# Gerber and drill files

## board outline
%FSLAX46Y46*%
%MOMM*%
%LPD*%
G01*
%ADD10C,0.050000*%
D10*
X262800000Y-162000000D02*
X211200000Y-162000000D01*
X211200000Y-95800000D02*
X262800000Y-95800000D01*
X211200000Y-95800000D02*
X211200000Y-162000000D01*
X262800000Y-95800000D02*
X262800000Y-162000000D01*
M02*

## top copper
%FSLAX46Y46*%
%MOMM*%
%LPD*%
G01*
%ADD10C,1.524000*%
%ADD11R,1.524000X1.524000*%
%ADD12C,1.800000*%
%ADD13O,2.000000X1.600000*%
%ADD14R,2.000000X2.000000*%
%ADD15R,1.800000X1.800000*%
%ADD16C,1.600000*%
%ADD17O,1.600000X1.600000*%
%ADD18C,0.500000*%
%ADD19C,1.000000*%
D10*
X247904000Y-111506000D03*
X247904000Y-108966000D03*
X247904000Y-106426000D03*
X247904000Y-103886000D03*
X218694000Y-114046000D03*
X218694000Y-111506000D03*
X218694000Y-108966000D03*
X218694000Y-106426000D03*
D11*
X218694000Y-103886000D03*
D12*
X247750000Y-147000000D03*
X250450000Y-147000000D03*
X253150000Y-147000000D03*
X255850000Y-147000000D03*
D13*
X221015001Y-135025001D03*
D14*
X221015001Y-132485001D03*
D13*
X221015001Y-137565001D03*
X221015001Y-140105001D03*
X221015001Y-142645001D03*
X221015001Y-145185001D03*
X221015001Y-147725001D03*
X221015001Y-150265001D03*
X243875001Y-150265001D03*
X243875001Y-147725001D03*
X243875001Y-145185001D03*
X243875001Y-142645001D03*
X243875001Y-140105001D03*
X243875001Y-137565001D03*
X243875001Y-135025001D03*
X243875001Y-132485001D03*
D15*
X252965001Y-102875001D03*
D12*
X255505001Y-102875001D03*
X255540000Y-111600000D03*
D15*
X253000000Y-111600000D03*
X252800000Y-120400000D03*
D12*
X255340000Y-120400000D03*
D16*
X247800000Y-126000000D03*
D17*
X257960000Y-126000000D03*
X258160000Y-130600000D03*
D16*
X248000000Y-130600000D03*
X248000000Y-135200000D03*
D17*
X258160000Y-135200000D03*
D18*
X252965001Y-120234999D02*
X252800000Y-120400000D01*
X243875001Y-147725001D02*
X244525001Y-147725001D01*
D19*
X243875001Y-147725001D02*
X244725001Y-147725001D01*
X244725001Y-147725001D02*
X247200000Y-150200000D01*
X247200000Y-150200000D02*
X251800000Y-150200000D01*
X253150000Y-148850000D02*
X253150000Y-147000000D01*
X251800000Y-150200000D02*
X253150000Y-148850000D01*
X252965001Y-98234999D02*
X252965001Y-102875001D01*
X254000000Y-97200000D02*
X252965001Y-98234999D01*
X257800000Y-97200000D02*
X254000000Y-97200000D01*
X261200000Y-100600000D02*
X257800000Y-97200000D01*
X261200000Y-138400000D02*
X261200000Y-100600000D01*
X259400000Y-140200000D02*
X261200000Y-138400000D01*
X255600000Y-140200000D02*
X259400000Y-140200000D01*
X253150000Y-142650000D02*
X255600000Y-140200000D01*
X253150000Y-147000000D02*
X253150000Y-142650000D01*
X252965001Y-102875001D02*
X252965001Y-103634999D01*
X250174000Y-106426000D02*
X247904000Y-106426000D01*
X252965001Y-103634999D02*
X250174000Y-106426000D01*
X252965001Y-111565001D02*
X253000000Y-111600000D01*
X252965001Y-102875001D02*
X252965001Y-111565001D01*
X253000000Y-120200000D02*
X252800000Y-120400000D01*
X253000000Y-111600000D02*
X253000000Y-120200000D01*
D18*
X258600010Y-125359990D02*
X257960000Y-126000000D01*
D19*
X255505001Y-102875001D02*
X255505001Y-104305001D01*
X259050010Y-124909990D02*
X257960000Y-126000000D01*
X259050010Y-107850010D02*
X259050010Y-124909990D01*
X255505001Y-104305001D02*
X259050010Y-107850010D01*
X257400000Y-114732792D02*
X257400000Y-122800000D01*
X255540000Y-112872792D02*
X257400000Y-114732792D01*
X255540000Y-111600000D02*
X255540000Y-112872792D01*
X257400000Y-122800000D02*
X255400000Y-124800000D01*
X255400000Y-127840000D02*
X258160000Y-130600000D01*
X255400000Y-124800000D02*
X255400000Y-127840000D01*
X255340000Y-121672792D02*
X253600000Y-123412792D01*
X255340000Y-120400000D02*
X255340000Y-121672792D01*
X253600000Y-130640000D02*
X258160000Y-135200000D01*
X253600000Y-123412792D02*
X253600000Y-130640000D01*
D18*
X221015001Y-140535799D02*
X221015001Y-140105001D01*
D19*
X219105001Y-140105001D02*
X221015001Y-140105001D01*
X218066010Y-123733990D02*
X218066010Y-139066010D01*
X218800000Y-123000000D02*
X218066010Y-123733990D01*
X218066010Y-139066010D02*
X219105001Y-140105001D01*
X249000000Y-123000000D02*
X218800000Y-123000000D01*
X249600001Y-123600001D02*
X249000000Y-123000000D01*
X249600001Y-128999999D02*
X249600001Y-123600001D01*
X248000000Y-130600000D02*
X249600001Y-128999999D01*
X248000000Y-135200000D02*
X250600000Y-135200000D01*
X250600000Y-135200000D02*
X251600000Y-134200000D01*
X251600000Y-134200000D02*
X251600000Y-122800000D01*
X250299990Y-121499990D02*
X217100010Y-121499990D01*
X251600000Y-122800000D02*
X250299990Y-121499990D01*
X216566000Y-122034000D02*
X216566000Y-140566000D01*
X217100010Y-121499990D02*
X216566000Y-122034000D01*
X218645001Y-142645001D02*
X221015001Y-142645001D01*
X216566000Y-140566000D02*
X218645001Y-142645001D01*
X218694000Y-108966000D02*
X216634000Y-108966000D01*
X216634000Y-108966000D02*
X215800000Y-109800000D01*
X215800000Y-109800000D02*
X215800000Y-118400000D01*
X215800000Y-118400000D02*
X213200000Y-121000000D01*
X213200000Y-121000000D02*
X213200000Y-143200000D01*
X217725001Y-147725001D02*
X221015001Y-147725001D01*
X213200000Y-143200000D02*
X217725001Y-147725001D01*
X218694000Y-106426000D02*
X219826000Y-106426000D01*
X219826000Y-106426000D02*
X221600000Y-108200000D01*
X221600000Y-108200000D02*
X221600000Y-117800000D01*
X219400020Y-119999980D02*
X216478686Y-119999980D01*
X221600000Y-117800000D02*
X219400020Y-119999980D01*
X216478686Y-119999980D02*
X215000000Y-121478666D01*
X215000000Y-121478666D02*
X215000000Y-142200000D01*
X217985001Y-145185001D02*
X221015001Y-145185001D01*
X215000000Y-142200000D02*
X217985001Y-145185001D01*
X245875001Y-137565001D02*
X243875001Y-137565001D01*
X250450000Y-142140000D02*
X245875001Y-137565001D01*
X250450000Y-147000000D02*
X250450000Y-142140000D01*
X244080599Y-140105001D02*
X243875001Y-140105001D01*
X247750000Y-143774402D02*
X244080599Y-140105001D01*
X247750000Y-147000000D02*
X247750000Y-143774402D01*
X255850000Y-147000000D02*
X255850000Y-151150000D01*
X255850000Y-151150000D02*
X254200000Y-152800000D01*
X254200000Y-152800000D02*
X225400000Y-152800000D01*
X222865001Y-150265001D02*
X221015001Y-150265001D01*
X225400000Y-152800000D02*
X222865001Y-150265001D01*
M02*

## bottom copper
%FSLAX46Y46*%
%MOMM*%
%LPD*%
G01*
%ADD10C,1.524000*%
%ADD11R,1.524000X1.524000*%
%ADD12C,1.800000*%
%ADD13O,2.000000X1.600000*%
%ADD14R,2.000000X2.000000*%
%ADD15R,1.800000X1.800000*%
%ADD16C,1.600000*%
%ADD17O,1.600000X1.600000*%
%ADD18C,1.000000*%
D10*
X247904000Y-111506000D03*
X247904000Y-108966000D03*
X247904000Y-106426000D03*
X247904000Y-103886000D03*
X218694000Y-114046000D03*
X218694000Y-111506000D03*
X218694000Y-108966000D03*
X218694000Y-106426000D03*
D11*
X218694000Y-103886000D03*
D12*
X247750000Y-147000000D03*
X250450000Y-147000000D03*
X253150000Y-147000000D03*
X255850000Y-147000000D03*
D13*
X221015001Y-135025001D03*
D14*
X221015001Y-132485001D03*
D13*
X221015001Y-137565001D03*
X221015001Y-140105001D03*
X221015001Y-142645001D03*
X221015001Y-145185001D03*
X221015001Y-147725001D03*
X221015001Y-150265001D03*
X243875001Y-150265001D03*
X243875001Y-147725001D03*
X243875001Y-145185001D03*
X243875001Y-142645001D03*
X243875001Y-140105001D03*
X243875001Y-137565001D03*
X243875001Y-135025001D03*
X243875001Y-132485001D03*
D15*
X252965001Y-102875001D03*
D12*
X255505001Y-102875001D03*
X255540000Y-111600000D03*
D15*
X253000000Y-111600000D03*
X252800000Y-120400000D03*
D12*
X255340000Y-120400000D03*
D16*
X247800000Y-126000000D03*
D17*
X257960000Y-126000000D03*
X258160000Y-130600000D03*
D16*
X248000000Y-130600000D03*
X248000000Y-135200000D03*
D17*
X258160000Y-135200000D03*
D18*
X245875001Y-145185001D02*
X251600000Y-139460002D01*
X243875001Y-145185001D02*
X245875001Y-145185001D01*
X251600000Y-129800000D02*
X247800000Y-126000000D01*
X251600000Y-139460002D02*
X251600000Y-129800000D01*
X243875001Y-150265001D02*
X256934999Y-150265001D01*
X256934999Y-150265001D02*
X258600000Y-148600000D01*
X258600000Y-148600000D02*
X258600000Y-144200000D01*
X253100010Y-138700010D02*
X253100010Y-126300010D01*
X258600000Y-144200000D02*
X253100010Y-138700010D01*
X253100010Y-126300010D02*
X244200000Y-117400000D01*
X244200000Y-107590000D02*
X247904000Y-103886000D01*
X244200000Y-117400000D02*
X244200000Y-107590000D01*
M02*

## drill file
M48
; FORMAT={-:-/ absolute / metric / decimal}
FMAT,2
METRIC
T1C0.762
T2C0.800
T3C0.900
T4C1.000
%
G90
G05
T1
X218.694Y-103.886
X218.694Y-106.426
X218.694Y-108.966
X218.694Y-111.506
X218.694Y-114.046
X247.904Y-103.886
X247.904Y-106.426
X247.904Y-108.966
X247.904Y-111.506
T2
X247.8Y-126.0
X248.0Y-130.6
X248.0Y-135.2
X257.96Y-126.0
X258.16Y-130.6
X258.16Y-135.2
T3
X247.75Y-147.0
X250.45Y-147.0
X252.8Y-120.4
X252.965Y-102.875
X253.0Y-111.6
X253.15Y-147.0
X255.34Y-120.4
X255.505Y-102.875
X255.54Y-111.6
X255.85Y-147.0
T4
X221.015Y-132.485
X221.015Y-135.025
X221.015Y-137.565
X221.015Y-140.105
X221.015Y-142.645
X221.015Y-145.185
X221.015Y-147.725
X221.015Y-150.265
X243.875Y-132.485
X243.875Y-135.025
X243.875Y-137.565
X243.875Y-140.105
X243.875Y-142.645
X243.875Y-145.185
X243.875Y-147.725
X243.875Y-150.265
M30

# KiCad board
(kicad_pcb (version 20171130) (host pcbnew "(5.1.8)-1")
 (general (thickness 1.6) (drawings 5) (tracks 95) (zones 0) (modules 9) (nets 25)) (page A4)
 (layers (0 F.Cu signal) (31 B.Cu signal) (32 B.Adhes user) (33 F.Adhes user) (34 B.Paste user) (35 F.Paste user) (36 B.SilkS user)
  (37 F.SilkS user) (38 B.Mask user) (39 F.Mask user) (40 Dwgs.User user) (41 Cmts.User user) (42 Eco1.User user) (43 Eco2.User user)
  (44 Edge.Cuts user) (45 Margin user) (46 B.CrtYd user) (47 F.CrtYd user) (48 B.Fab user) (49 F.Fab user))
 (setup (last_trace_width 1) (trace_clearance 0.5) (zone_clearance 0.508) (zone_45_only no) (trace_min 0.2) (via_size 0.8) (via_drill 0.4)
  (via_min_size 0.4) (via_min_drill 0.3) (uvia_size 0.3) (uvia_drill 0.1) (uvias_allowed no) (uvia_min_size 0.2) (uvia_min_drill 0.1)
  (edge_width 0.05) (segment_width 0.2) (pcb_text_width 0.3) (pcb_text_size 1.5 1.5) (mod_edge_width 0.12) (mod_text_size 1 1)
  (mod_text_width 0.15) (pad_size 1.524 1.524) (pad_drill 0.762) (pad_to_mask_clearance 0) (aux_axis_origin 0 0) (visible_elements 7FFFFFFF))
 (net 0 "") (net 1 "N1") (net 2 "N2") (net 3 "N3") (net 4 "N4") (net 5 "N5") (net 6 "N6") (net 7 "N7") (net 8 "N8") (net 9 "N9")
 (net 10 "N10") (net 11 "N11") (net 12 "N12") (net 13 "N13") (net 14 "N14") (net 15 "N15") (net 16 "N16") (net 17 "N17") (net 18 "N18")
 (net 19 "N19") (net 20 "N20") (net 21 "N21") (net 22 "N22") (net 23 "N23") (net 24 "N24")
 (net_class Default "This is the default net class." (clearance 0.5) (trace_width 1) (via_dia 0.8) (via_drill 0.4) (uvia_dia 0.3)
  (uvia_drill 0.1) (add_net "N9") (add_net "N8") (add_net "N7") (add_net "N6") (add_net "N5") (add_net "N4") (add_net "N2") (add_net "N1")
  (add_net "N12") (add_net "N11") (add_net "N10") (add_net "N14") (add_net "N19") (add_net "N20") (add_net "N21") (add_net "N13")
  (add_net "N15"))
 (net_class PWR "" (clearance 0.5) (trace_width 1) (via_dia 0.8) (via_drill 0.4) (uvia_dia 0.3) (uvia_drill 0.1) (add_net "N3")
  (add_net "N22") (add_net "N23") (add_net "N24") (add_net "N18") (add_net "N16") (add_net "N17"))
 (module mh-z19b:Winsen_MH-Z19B (layer F.Cu) (at 218.694 117.856 180)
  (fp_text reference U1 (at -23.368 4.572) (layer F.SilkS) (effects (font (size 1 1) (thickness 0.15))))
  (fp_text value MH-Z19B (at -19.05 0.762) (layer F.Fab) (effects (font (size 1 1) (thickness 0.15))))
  (pad 9 thru_hole circle (at -29.21 6.35 180) (size 1.524 1.524) (drill 0.762) (layers *.Cu *.Mask) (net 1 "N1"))
  (pad 8 thru_hole circle (at -29.21 8.89 180) (size 1.524 1.524) (drill 0.762) (layers *.Cu *.Mask) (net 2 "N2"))
  (pad 7 thru_hole circle (at -29.21 11.43 180) (size 1.524 1.524) (drill 0.762) (layers *.Cu *.Mask) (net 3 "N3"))
  (pad 6 thru_hole circle (at -29.21 13.97 180) (size 1.524 1.524) (drill 0.762) (layers *.Cu *.Mask) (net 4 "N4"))
  (pad 5 thru_hole circle (at 0 3.81 180) (size 1.524 1.524) (drill 0.762) (layers *.Cu *.Mask) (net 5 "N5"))
  (pad 4 thru_hole circle (at 0 6.35 180) (size 1.524 1.524) (drill 0.762) (layers *.Cu *.Mask) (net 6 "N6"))
  (pad 3 thru_hole circle (at 0 8.89 180) (size 1.524 1.524) (drill 0.762) (layers *.Cu *.Mask) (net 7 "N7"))
  (pad 2 thru_hole circle (at 0 11.43 180) (size 1.524 1.524) (drill 0.762) (layers *.Cu *.Mask) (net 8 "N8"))
  (pad 1 thru_hole rect (at 0 13.97 180) (size 1.524 1.524) (drill 0.762) (layers *.Cu *.Mask) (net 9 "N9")))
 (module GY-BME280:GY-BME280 (layer F.Cu) (at 251.8 149 180)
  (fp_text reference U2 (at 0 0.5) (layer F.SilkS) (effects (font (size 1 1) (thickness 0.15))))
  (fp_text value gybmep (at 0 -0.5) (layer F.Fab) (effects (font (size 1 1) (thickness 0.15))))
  (pad 4 thru_hole circle (at 4.05 2 180) (size 1.8 1.8) (drill 0.9) (layers *.Cu *.Mask) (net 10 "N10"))
  (pad 3 thru_hole circle (at 1.35 2 180) (size 1.8 1.8) (drill 0.9) (layers *.Cu *.Mask) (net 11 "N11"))
  (pad 2 thru_hole circle (at -1.35 2 180) (size 1.8 1.8) (drill 0.9) (layers *.Cu *.Mask) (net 3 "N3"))
  (pad 1 thru_hole circle (at -4.05 2 180) (size 1.8 1.8) (drill 0.9) (layers *.Cu *.Mask) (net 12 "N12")))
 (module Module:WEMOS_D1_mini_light (layer F.Cu) (at 221.015001 132.485001)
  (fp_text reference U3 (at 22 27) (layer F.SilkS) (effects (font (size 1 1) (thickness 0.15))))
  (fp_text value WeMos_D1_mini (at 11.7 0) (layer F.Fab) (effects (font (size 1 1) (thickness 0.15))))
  (pad 2 thru_hole oval (at 0 2.54) (size 2 1.6) (drill 1) (layers *.Cu *.Mask) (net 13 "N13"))
  (pad 1 thru_hole rect (at 0 0) (size 2 2) (drill 1) (layers *.Cu *.Mask) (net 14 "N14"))
  (pad 3 thru_hole oval (at 0 5.08) (size 2 1.6) (drill 1) (layers *.Cu *.Mask) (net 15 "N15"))
  (pad 4 thru_hole oval (at 0 7.62) (size 2 1.6) (drill 1) (layers *.Cu *.Mask) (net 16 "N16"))
  (pad 5 thru_hole oval (at 0 10.16) (size 2 1.6) (drill 1) (layers *.Cu *.Mask) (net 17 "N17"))
  (pad 6 thru_hole oval (at 0 12.7) (size 2 1.6) (drill 1) (layers *.Cu *.Mask) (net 8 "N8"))
  (pad 7 thru_hole oval (at 0 15.24) (size 2 1.6) (drill 1) (layers *.Cu *.Mask) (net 7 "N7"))
  (pad 8 thru_hole oval (at 0 17.78) (size 2 1.6) (drill 1) (layers *.Cu *.Mask) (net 12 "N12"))
  (pad 9 thru_hole oval (at 22.86 17.78) (size 2 1.6) (drill 1) (layers *.Cu *.Mask) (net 4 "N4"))
  (pad 10 thru_hole oval (at 22.86 15.24) (size 2 1.6) (drill 1) (layers *.Cu *.Mask) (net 3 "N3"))
  (pad 11 thru_hole oval (at 22.86 12.7) (size 2 1.6) (drill 1) (layers *.Cu *.Mask) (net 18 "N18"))
  (pad 12 thru_hole oval (at 22.86 10.16) (size 2 1.6) (drill 1) (layers *.Cu *.Mask) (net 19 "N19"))
  (pad 13 thru_hole oval (at 22.86 7.62) (size 2 1.6) (drill 1) (layers *.Cu *.Mask) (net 10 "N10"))
  (pad 14 thru_hole oval (at 22.86 5.08) (size 2 1.6) (drill 1) (layers *.Cu *.Mask) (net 11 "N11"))
  (pad 15 thru_hole oval (at 22.86 2.54) (size 2 1.6) (drill 1) (layers *.Cu *.Mask) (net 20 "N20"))
  (pad 16 thru_hole oval (at 22.86 0) (size 2 1.6) (drill 1) (layers *.Cu *.Mask) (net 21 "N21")))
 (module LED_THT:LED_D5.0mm (layer F.Cu) (at 252.965001 102.875001)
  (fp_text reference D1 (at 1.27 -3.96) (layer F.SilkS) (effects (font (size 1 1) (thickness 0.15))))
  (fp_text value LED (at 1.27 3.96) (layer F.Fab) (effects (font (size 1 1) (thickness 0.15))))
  (pad 1 thru_hole rect (at 0 0) (size 1.8 1.8) (drill 0.9) (layers *.Cu *.Mask) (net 3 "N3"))
  (pad 2 thru_hole circle (at 2.54 0) (size 1.8 1.8) (drill 0.9) (layers *.Cu *.Mask) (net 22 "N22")))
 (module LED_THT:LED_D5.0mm (layer F.Cu) (at 253 111.6)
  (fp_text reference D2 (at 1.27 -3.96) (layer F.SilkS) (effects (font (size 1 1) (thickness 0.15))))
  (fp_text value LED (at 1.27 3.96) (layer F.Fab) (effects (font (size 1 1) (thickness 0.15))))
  (pad 2 thru_hole circle (at 2.54 0) (size 1.8 1.8) (drill 0.9) (layers *.Cu *.Mask) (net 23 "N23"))
  (pad 1 thru_hole rect (at 0 0) (size 1.8 1.8) (drill 0.9) (layers *.Cu *.Mask) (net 3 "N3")))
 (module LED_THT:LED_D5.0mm (layer F.Cu) (at 252.8 120.4)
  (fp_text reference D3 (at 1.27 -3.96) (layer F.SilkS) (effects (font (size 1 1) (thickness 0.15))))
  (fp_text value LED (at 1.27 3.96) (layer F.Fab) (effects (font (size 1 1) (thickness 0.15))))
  (pad 1 thru_hole rect (at 0 0) (size 1.8 1.8) (drill 0.9) (layers *.Cu *.Mask) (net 3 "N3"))
  (pad 2 thru_hole circle (at 2.54 0) (size 1.8 1.8) (drill 0.9) (layers *.Cu *.Mask) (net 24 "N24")))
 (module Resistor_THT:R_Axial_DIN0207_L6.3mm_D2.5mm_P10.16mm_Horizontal (layer F.Cu) (at 247.8 126)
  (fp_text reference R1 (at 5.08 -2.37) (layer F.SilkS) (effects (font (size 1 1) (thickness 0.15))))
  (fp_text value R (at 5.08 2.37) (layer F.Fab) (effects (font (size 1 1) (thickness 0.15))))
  (pad 1 thru_hole circle (at 0 0) (size 1.6 1.6) (drill 0.8) (layers *.Cu *.Mask) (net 18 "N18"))
  (pad 2 thru_hole oval (at 10.16 0) (size 1.6 1.6) (drill 0.8) (layers *.Cu *.Mask) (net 22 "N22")))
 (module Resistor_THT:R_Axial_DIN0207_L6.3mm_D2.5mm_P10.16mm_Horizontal (layer F.Cu) (at 248 130.6)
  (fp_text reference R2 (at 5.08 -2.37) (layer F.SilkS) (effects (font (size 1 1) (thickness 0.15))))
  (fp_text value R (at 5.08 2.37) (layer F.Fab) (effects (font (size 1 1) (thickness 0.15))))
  (pad 2 thru_hole oval (at 10.16 0) (size 1.6 1.6) (drill 0.8) (layers *.Cu *.Mask) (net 23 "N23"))
  (pad 1 thru_hole circle (at 0 0) (size 1.6 1.6) (drill 0.8) (layers *.Cu *.Mask) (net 16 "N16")))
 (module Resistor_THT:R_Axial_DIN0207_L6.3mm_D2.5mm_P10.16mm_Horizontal (layer F.Cu) (at 248 135.2)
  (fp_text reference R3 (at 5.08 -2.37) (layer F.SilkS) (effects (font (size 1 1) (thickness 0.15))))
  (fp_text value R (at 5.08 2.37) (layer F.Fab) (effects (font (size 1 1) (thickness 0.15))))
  (pad 1 thru_hole circle (at 0 0) (size 1.6 1.6) (drill 0.8) (layers *.Cu *.Mask) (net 17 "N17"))
  (pad 2 thru_hole oval (at 10.16 0) (size 1.6 1.6) (drill 0.8) (layers *.Cu *.Mask) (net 24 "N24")))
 (gr_line (start 262.8 162) (end 211.2 162) (layer Edge.Cuts) (width 0.05))
 (gr_line (start 211.2 95.8) (end 262.8 95.8) (layer Edge.Cuts) (width 0.05))
 (gr_line (start 211.2 95.8) (end 211.2 162) (layer Edge.Cuts) (width 0.05))
 (gr_line (start 262.8 95.8) (end 262.8 162) (layer Edge.Cuts) (width 0.05))
 (segment (start 252.965001 120.234999) (end 252.8 120.4) (width 0.5) (layer F.Cu) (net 3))
 (segment (start 243.875001 147.725001) (end 244.525001 147.725001) (width 0.5) (layer F.Cu) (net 3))
 (segment (start 243.875001 147.725001) (end 244.725001 147.725001) (width 1) (layer F.Cu) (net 3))
 (segment (start 244.725001 147.725001) (end 247.2 150.2) (width 1) (layer F.Cu) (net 3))
 (segment (start 247.2 150.2) (end 251.8 150.2) (width 1) (layer F.Cu) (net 3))
 (segment (start 253.15 148.85) (end 253.15 147) (width 1) (layer F.Cu) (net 3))
 (segment (start 251.8 150.2) (end 253.15 148.85) (width 1) (layer F.Cu) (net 3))
 (segment (start 252.965001 98.234999) (end 252.965001 102.875001) (width 1) (layer F.Cu) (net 3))
 (segment (start 254 97.2) (end 252.965001 98.234999) (width 1) (layer F.Cu) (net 3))
 (segment (start 257.8 97.2) (end 254 97.2) (width 1) (layer F.Cu) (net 3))
 (segment (start 261.2 100.6) (end 257.8 97.2) (width 1) (layer F.Cu) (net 3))
 (segment (start 261.2 138.4) (end 261.2 100.6) (width 1) (layer F.Cu) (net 3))
 (segment (start 259.4 140.2) (end 261.2 138.4) (width 1) (layer F.Cu) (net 3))
 (segment (start 255.6 140.2) (end 259.4 140.2) (width 1) (layer F.Cu) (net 3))
 (segment (start 253.15 142.65) (end 255.6 140.2) (width 1) (layer F.Cu) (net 3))
 (segment (start 253.15 147) (end 253.15 142.65) (width 1) (layer F.Cu) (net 3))
 (segment (start 252.965001 102.875001) (end 252.965001 103.634999) (width 1) (layer F.Cu) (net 3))
 (segment (start 250.174 106.426) (end 247.904 106.426) (width 1) (layer F.Cu) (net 3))
 (segment (start 252.965001 103.634999) (end 250.174 106.426) (width 1) (layer F.Cu) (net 3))
 (segment (start 252.965001 111.565001) (end 253 111.6) (width 1) (layer F.Cu) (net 3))
 (segment (start 252.965001 102.875001) (end 252.965001 111.565001) (width 1) (layer F.Cu) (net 3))
 (segment (start 253 120.2) (end 252.8 120.4) (width 1) (layer F.Cu) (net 3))
 (segment (start 253 111.6) (end 253 120.2) (width 1) (layer F.Cu) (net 3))
 (segment (start 258.60001 125.35999) (end 257.96 126) (width 0.5) (layer F.Cu) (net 22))
 (segment (start 255.505001 102.875001) (end 255.505001 104.305001) (width 1) (layer F.Cu) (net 22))
 (segment (start 259.05001 124.90999) (end 257.96 126) (width 1) (layer F.Cu) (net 22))
 (segment (start 259.05001 107.85001) (end 259.05001 124.90999) (width 1) (layer F.Cu) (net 22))
 (segment (start 255.505001 104.305001) (end 259.05001 107.85001) (width 1) (layer F.Cu) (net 22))
 (segment (start 257.4 114.732792) (end 257.4 122.8) (width 1) (layer F.Cu) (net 23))
 (segment (start 255.54 112.872792) (end 257.4 114.732792) (width 1) (layer F.Cu) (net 23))
 (segment (start 255.54 111.6) (end 255.54 112.872792) (width 1) (layer F.Cu) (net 23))
 (segment (start 257.4 122.8) (end 255.4 124.8) (width 1) (layer F.Cu) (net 23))
 (segment (start 255.4 127.84) (end 258.16 130.6) (width 1) (layer F.Cu) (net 23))
 (segment (start 255.4 124.8) (end 255.4 127.84) (width 1) (layer F.Cu) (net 23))
 (segment (start 255.34 121.672792) (end 253.6 123.412792) (width 1) (layer F.Cu) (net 24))
 (segment (start 255.34 120.4) (end 255.34 121.672792) (width 1) (layer F.Cu) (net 24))
 (segment (start 253.6 130.64) (end 258.16 135.2) (width 1) (layer F.Cu) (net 24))
 (segment (start 253.6 123.412792) (end 253.6 130.64) (width 1) (layer F.Cu) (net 24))
 (segment (start 245.875001 145.185001) (end 251.6 139.460002) (width 1) (layer B.Cu) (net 18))
 (segment (start 243.875001 145.185001) (end 245.875001 145.185001) (width 1) (layer B.Cu) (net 18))
 (segment (start 251.6 129.8) (end 247.8 126) (width 1) (layer B.Cu) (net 18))
 (segment (start 251.6 139.460002) (end 251.6 129.8) (width 1) (layer B.Cu) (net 18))
 (segment (start 221.015001 140.535799) (end 221.015001 140.105001) (width 0.5) (layer F.Cu) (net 16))
 (segment (start 219.105001 140.105001) (end 221.015001 140.105001) (width 1) (layer F.Cu) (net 16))
 (segment (start 218.06601 123.73399) (end 218.06601 139.06601) (width 1) (layer F.Cu) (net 16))
 (segment (start 218.8 123) (end 218.06601 123.73399) (width 1) (layer F.Cu) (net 16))
 (segment (start 218.06601 139.06601) (end 219.105001 140.105001) (width 1) (layer F.Cu) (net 16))
 (segment (start 249 123) (end 218.8 123) (width 1) (layer F.Cu) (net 16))
 (segment (start 249.600001 123.600001) (end 249 123) (width 1) (layer F.Cu) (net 16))
 (segment (start 249.600001 128.999999) (end 249.600001 123.600001) (width 1) (layer F.Cu) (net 16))
 (segment (start 248 130.6) (end 249.600001 128.999999) (width 1) (layer F.Cu) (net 16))
 (segment (start 248 135.2) (end 250.6 135.2) (width 1) (layer F.Cu) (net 17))
 (segment (start 250.6 135.2) (end 251.6 134.2) (width 1) (layer F.Cu) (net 17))
 (segment (start 251.6 134.2) (end 251.6 122.8) (width 1) (layer F.Cu) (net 17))
 (segment (start 250.29999 121.49999) (end 217.10001 121.49999) (width 1) (layer F.Cu) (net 17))
 (segment (start 251.6 122.8) (end 250.29999 121.49999) (width 1) (layer F.Cu) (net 17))
 (segment (start 216.566 122.034) (end 216.566 140.566) (width 1) (layer F.Cu) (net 17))
 (segment (start 217.10001 121.49999) (end 216.566 122.034) (width 1) (layer F.Cu) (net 17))
 (segment (start 218.645001 142.645001) (end 221.015001 142.645001) (width 1) (layer F.Cu) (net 17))
 (segment (start 216.566 140.566) (end 218.645001 142.645001) (width 1) (layer F.Cu) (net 17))
 (segment (start 243.875001 150.265001) (end 256.934999 150.265001) (width 1) (layer B.Cu) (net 4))
 (segment (start 256.934999 150.265001) (end 258.6 148.6) (width 1) (layer B.Cu) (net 4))
 (segment (start 258.6 148.6) (end 258.6 144.2) (width 1) (layer B.Cu) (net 4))
 (segment (start 253.10001 138.70001) (end 253.10001 126.30001) (width 1) (layer B.Cu) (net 4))
 (segment (start 258.6 144.2) (end 253.10001 138.70001) (width 1) (layer B.Cu) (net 4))
 (segment (start 253.10001 126.30001) (end 244.2 117.4) (width 1) (layer B.Cu) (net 4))
 (segment (start 244.2 107.59) (end 247.904 103.886) (width 1) (layer B.Cu) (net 4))
 (segment (start 244.2 117.4) (end 244.2 107.59) (width 1) (layer B.Cu) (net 4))
 (segment (start 218.694 108.966) (end 216.634 108.966) (width 1) (layer F.Cu) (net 7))
 (segment (start 216.634 108.966) (end 215.8 109.8) (width 1) (layer F.Cu) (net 7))
 (segment (start 215.8 109.8) (end 215.8 118.4) (width 1) (layer F.Cu) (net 7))
 (segment (start 215.8 118.4) (end 213.2 121) (width 1) (layer F.Cu) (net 7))
 (segment (start 213.2 121) (end 213.2 143.2) (width 1) (layer F.Cu) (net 7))
 (segment (start 217.725001 147.725001) (end 221.015001 147.725001) (width 1) (layer F.Cu) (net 7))
 (segment (start 213.2 143.2) (end 217.725001 147.725001) (width 1) (layer F.Cu) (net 7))
 (segment (start 218.694 106.426) (end 219.826 106.426) (width 1) (layer F.Cu) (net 8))
 (segment (start 219.826 106.426) (end 221.6 108.2) (width 1) (layer F.Cu) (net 8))
 (segment (start 221.6 108.2) (end 221.6 117.8) (width 1) (layer F.Cu) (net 8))
 (segment (start 219.40002 119.99998) (end 216.478686 119.99998) (width 1) (layer F.Cu) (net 8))
 (segment (start 221.6 117.8) (end 219.40002 119.99998) (width 1) (layer F.Cu) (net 8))
 (segment (start 216.478686 119.99998) (end 215 121.478666) (width 1) (layer F.Cu) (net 8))
 (segment (start 215 121.478666) (end 215 142.2) (width 1) (layer F.Cu) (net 8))
 (segment (start 217.985001 145.185001) (end 221.015001 145.185001) (width 1) (layer F.Cu) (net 8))
 (segment (start 215 142.2) (end 217.985001 145.185001) (width 1) (layer F.Cu) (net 8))
 (segment (start 245.875001 137.565001) (end 243.875001 137.565001) (width 1) (layer F.Cu) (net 11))
 (segment (start 250.45 142.14) (end 245.875001 137.565001) (width 1) (layer F.Cu) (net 11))
 (segment (start 250.45 147) (end 250.45 142.14) (width 1) (layer F.Cu) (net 11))
 (segment (start 244.080599 140.105001) (end 243.875001 140.105001) (width 1) (layer F.Cu) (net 10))
 (segment (start 247.75 143.774402) (end 244.080599 140.105001) (width 1) (layer F.Cu) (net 10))
 (segment (start 247.75 147) (end 247.75 143.774402) (width 1) (layer F.Cu) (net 10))
 (segment (start 255.85 147) (end 255.85 151.15) (width 1) (layer F.Cu) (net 12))
 (segment (start 255.85 151.15) (end 254.2 152.8) (width 1) (layer F.Cu) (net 12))
 (segment (start 254.2 152.8) (end 225.4 152.8) (width 1) (layer F.Cu) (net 12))
 (segment (start 222.865001 150.265001) (end 221.015001 150.265001) (width 1) (layer F.Cu) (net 12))
 (segment (start 225.4 152.8) (end 222.865001 150.265001) (width 1) (layer F.Cu) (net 12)))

